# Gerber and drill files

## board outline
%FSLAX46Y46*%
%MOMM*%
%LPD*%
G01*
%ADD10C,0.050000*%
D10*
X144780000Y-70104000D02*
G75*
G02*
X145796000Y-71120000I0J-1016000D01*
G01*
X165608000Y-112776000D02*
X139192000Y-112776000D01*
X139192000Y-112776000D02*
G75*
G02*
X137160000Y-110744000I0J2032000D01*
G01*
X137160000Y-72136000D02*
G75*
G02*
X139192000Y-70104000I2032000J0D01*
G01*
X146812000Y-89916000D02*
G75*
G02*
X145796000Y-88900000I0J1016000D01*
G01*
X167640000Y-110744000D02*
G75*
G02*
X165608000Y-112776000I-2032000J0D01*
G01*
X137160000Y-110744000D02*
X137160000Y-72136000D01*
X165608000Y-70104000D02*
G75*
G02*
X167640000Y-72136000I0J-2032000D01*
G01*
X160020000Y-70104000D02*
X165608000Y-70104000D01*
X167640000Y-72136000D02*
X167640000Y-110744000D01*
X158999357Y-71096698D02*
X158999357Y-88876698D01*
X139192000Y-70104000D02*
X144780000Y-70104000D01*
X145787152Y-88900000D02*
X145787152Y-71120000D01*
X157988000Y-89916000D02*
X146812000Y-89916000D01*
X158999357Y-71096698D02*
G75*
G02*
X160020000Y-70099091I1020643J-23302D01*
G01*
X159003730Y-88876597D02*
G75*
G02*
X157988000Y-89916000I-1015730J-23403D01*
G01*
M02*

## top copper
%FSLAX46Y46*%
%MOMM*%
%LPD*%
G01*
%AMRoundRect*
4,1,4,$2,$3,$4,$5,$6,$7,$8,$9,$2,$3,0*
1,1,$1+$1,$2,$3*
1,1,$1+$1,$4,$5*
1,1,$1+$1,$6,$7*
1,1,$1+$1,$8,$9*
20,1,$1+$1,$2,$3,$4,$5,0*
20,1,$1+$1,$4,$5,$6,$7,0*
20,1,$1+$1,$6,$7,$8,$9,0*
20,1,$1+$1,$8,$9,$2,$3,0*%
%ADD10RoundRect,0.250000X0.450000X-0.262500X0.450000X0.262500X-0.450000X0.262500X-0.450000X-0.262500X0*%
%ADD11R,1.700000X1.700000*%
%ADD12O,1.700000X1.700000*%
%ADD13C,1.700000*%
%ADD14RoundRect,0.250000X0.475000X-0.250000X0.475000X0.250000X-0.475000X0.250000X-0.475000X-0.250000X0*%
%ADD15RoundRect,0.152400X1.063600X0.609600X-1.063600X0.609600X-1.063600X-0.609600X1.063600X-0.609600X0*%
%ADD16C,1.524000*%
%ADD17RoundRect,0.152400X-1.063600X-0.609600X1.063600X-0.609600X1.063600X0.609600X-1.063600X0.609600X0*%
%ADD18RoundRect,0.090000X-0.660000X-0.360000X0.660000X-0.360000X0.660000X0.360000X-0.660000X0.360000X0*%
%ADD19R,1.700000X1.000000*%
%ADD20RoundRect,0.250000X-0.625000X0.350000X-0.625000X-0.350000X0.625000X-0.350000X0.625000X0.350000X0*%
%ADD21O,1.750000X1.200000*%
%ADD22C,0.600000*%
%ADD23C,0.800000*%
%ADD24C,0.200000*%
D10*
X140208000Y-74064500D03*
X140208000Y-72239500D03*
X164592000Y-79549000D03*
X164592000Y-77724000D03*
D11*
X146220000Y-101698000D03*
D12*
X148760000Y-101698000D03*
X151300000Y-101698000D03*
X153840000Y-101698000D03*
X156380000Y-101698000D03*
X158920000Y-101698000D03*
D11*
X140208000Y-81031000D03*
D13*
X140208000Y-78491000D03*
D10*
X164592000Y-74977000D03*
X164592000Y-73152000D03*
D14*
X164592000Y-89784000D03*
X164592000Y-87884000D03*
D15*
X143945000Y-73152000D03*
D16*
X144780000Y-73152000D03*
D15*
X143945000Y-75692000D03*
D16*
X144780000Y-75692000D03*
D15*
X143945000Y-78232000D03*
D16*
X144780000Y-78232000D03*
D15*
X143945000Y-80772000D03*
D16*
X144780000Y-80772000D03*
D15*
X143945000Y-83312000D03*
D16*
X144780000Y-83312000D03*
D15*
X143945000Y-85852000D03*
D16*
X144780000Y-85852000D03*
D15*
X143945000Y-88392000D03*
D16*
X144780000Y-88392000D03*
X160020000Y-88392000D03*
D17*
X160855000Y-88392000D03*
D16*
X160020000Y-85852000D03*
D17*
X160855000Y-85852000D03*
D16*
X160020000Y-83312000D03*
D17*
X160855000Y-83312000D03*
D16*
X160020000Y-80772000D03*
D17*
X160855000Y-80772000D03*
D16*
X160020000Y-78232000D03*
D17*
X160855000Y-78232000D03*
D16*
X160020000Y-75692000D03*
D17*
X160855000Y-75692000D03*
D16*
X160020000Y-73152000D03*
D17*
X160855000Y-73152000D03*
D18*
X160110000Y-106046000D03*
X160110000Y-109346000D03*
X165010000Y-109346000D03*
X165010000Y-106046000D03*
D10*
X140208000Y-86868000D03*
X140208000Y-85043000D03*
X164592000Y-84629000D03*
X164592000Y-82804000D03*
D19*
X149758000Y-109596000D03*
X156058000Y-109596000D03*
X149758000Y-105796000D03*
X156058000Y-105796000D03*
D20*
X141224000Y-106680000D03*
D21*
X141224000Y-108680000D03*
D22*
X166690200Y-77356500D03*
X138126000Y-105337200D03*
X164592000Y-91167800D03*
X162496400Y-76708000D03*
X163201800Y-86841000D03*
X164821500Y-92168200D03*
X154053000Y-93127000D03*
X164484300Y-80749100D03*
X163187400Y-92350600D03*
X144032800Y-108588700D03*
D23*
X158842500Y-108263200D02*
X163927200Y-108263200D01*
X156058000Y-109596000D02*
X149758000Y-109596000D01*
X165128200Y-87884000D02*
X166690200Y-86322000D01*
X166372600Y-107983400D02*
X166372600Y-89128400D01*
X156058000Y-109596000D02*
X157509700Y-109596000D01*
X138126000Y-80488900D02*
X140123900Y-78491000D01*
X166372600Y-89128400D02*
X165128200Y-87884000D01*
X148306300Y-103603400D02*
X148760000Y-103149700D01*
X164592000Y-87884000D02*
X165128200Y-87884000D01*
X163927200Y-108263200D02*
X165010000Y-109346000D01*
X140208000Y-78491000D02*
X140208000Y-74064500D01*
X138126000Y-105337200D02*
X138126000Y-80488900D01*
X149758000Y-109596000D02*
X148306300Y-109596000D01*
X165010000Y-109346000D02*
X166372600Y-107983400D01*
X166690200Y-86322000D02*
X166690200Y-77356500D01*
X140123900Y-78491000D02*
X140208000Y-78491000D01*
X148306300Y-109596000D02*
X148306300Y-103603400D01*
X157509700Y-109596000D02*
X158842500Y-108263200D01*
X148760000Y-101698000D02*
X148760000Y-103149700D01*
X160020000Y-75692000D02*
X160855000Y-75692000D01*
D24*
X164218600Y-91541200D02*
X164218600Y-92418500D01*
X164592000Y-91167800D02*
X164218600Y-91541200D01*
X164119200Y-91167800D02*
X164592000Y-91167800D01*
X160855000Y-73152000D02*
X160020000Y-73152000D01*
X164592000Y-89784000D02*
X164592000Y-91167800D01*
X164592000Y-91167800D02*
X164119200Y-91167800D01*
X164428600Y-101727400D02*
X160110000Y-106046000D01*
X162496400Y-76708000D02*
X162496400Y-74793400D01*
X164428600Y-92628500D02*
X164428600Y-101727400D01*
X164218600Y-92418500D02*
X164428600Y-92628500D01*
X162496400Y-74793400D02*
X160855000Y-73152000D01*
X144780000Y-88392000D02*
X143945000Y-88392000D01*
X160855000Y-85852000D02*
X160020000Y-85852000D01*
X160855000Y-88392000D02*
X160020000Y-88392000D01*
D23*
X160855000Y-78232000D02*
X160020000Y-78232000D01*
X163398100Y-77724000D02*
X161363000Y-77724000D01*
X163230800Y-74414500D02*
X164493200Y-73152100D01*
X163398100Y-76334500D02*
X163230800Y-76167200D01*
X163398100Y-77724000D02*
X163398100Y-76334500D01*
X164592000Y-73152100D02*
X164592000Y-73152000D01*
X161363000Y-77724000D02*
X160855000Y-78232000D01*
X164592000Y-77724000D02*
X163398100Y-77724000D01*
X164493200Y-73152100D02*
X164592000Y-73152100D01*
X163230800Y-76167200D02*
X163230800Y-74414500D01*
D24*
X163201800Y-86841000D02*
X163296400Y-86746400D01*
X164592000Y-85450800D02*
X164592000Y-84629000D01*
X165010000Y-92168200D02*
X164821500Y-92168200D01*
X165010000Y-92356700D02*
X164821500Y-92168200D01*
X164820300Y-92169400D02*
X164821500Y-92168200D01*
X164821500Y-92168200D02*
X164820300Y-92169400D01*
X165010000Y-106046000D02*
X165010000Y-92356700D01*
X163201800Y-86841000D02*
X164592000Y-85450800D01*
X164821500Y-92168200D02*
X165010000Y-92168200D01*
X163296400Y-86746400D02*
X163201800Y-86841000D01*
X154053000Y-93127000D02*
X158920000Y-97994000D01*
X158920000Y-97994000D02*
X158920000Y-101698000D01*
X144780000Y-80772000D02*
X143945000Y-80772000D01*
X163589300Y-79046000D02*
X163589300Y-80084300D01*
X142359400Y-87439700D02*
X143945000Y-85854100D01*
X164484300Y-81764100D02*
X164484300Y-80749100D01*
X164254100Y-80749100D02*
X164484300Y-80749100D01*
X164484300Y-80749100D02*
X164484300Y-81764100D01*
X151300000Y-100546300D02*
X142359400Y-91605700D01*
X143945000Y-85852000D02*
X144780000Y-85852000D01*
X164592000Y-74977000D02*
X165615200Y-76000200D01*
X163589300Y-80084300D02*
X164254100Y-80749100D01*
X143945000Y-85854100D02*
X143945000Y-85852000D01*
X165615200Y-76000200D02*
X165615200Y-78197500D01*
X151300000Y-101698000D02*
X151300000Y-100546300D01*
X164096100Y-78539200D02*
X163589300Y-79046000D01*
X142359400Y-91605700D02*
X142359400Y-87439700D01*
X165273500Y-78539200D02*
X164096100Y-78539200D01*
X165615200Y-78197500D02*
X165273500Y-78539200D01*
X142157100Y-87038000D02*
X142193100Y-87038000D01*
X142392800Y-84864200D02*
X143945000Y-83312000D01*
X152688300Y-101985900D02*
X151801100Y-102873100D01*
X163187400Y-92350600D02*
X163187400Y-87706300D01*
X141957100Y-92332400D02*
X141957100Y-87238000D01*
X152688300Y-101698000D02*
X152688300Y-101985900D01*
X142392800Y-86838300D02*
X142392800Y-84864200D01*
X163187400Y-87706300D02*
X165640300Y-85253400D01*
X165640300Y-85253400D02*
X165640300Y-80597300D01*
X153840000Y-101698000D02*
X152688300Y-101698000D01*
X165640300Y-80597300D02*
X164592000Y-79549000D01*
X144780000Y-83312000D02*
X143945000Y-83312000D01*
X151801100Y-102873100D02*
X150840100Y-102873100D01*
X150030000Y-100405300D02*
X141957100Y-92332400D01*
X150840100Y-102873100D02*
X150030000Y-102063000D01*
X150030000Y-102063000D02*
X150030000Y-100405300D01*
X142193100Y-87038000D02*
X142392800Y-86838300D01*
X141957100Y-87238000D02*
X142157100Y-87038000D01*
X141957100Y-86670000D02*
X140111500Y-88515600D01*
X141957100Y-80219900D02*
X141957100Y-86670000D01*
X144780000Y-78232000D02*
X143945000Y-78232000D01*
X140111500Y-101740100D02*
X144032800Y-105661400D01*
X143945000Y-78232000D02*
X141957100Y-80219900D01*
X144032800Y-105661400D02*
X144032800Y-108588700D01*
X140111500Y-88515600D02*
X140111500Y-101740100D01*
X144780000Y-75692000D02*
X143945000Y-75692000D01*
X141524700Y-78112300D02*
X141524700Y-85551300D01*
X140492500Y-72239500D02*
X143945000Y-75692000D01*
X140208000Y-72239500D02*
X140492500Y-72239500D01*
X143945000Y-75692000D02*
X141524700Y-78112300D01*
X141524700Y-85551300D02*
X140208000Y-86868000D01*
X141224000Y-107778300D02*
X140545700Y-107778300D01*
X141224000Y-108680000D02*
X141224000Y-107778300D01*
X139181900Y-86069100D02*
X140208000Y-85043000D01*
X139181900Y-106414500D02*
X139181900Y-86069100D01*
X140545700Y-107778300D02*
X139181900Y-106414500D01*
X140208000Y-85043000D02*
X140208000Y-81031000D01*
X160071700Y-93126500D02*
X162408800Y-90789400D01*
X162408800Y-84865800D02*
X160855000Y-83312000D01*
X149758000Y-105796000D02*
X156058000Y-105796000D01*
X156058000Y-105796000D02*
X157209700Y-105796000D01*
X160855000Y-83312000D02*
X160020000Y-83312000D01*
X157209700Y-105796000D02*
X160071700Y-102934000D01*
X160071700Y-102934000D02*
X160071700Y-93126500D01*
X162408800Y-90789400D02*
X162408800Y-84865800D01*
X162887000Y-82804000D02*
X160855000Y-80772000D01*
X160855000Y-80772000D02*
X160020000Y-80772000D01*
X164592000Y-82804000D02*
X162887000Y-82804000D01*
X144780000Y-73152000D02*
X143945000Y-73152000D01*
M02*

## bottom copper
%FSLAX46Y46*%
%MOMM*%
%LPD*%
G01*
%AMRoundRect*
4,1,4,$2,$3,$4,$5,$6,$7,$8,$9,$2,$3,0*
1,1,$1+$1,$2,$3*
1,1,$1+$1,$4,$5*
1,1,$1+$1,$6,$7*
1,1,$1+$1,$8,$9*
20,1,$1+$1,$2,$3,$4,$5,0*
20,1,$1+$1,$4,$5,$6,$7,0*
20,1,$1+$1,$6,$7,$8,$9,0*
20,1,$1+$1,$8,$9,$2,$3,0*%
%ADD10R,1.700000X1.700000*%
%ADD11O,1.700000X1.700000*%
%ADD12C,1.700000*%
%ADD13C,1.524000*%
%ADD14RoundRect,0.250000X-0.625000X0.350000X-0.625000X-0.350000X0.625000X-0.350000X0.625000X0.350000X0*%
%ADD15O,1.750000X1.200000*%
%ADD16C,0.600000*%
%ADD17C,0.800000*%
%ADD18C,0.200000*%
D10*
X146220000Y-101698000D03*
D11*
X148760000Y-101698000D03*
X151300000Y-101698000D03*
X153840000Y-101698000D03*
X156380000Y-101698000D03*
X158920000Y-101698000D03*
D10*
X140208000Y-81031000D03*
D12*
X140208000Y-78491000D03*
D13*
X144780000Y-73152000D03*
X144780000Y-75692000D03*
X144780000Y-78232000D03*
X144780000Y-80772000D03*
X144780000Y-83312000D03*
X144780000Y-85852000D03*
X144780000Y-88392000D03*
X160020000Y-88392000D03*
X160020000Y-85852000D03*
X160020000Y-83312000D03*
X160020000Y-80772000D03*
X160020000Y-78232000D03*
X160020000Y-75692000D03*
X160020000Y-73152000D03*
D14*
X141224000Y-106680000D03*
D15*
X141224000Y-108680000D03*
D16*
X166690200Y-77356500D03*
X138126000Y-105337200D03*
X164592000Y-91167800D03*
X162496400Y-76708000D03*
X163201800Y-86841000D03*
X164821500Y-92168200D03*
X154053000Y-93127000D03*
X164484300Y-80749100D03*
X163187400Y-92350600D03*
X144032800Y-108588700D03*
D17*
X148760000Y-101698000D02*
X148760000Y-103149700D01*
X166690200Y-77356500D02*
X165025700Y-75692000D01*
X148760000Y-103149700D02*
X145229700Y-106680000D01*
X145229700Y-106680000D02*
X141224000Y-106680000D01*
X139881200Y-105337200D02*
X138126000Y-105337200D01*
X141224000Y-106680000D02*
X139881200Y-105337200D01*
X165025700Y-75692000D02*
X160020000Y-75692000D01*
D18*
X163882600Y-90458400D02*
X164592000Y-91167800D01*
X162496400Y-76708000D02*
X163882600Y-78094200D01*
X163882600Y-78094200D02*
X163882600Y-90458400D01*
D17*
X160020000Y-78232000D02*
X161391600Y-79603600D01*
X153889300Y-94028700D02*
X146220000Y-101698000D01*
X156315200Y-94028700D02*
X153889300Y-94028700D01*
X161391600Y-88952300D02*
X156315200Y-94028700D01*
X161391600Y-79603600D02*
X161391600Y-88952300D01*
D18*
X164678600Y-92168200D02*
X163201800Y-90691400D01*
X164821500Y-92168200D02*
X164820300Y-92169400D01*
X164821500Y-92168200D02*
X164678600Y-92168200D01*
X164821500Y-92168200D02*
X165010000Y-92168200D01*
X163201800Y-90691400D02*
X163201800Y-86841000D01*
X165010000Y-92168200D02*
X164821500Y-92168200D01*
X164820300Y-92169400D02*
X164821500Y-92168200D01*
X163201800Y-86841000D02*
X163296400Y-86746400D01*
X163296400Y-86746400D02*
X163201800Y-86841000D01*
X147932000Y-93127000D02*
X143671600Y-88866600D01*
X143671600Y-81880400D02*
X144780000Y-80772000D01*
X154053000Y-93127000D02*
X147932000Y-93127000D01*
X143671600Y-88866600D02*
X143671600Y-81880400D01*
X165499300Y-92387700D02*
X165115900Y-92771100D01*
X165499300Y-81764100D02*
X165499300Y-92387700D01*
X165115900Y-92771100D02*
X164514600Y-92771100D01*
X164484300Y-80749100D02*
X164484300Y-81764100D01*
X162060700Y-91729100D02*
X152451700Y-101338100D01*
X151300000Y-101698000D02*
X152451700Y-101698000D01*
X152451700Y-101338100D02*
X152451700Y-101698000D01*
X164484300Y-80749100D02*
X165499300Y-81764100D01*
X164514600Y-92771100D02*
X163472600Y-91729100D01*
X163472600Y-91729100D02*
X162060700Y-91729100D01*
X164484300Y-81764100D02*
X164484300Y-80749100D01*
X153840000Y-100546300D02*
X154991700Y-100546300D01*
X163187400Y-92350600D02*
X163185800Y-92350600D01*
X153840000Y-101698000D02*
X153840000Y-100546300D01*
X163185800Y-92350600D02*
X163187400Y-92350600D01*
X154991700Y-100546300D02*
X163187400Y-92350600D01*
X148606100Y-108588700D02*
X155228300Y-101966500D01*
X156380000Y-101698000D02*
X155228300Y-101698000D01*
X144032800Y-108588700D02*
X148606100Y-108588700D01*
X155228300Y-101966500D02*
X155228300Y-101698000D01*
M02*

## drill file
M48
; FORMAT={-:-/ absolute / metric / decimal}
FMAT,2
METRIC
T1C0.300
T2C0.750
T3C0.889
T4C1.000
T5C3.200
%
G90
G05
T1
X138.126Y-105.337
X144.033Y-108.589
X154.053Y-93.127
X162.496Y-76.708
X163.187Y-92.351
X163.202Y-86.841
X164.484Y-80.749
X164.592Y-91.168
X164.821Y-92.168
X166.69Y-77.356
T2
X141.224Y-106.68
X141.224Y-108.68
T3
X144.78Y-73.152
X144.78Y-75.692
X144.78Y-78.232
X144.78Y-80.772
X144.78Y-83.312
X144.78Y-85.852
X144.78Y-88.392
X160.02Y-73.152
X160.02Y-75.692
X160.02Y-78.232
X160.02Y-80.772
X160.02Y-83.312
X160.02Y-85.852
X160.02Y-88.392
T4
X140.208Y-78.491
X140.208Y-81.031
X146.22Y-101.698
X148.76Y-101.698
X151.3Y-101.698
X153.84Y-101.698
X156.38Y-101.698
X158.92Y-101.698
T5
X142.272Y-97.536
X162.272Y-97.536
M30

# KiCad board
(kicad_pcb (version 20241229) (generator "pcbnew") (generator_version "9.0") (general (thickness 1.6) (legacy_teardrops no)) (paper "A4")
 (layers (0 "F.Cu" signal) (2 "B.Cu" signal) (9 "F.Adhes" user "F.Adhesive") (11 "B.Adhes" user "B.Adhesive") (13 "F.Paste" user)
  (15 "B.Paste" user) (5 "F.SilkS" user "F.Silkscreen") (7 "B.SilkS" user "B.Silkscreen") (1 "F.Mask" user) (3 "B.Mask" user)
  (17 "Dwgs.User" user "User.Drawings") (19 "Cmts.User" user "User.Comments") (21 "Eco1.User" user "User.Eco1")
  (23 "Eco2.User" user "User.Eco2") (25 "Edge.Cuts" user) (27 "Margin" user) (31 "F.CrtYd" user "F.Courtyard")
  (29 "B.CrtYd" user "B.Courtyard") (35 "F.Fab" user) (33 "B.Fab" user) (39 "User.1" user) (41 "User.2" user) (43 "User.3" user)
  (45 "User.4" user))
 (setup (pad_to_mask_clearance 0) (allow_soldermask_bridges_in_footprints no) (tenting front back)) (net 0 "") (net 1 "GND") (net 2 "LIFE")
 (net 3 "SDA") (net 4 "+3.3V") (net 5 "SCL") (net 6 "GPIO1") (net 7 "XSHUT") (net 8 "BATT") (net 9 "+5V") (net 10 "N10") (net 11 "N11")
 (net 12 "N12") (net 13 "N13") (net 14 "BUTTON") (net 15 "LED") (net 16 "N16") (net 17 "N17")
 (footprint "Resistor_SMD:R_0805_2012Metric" (layer "F.Cu") (at 140.208 73.152 90)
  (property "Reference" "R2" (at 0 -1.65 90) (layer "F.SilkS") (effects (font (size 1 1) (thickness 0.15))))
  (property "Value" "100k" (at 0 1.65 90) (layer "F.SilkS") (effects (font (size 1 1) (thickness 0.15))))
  (pad "1" smd roundrect (at -0.9125 0 90) (size 1.025 1.4) (layers "F.Cu" "F.Mask" "F.Paste") (roundrect_rratio 0.243902) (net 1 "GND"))
  (pad "2" smd roundrect (at 0.9125 0 90) (size 1.025 1.4) (layers "F.Cu" "F.Mask" "F.Paste") (roundrect_rratio 0.243902) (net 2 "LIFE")))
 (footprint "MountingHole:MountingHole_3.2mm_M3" (layer "F.Cu") (at 162.272 97.536)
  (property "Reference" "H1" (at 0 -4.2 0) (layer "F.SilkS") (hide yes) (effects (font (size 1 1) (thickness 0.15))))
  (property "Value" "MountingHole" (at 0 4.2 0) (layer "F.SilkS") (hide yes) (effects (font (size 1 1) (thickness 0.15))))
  (pad "" np_thru_hole circle (at 0 0) (size 3.2 3.2) (drill 3.2) (layers "*.Cu" "*.Mask")))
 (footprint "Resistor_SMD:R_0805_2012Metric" (layer "F.Cu") (at 164.592 78.6365 90)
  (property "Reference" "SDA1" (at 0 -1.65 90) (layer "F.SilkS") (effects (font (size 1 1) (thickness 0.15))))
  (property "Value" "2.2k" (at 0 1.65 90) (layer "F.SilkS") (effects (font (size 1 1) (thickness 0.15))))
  (pad "1" smd roundrect (at -0.9125 0 90) (size 1.025 1.4) (layers "F.Cu" "F.Mask" "F.Paste") (roundrect_rratio 0.243902) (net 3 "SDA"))
  (pad "2" smd roundrect (at 0.9125 0 90) (size 1.025 1.4) (layers "F.Cu" "F.Mask" "F.Paste") (roundrect_rratio 0.243902) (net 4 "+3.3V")))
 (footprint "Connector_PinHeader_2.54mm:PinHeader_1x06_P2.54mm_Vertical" (layer "F.Cu") (at 146.22 101.698 90)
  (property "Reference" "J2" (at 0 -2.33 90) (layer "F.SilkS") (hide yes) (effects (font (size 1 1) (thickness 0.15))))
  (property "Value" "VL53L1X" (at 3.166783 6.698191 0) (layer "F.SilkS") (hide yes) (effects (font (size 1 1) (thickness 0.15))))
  (pad "1" thru_hole rect (at 0 0 90) (size 1.7 1.7) (drill 1) (layers "*.Cu" "*.Mask") (remove_unused_layers no) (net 4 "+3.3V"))
  (pad "2" thru_hole oval (at 0 2.54 90) (size 1.7 1.7) (drill 1) (layers "*.Cu" "*.Mask") (remove_unused_layers no) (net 1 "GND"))
  (pad "3" thru_hole oval (at 0 5.08 90) (size 1.7 1.7) (drill 1) (layers "*.Cu" "*.Mask") (remove_unused_layers no) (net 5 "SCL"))
  (pad "4" thru_hole oval (at 0 7.62 90) (size 1.7 1.7) (drill 1) (layers "*.Cu" "*.Mask") (remove_unused_layers no) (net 3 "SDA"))
  (pad "5" thru_hole oval (at 0 10.16 90) (size 1.7 1.7) (drill 1) (layers "*.Cu" "*.Mask") (remove_unused_layers no) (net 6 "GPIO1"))
  (pad "6" thru_hole oval (at 0 12.7 90) (size 1.7 1.7) (drill 1) (layers "*.Cu" "*.Mask") (remove_unused_layers no) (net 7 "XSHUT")))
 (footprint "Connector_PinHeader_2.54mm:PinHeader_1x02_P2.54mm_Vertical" (layer "F.Cu") (at 140.208 81.031 180)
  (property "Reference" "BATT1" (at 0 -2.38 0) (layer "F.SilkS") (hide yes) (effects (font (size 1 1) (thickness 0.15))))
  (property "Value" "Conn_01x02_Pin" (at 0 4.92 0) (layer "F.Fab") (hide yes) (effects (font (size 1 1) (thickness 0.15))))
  (pad "1" thru_hole rect (at 0 0 180) (size 1.7 1.7) (drill 1) (layers "*.Cu" "*.Mask") (remove_unused_layers no) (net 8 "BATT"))
  (pad "2" thru_hole circle (at 0 2.54 180) (size 1.7 1.7) (drill 1) (layers "*.Cu" "*.Mask") (remove_unused_layers no) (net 1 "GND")))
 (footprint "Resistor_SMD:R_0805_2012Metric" (layer "F.Cu") (at 164.592 74.0645 90)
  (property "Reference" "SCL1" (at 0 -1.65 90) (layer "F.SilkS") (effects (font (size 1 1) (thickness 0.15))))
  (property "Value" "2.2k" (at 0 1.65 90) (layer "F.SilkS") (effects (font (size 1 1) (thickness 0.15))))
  (pad "1" smd roundrect (at -0.9125 0 90) (size 1.025 1.4) (layers "F.Cu" "F.Mask" "F.Paste") (roundrect_rratio 0.243902) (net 5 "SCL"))
  (pad "2" smd roundrect (at 0.9125 0 90) (size 1.025 1.4) (layers "F.Cu" "F.Mask" "F.Paste") (roundrect_rratio 0.243902) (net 4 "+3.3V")))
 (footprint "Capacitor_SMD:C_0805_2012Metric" (layer "F.Cu") (at 164.592 88.834 90)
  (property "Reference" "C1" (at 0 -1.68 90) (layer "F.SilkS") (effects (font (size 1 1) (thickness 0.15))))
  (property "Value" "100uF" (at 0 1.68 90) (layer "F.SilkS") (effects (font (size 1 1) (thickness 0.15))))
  (pad "1" smd roundrect (at -0.95 0 90) (size 1 1.45) (layers "F.Cu" "F.Mask" "F.Paste") (roundrect_rratio 0.25) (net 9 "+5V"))
  (pad "2" smd roundrect (at 0.95 0 90) (size 1 1.45) (layers "F.Cu" "F.Mask" "F.Paste") (roundrect_rratio 0.25) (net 1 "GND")))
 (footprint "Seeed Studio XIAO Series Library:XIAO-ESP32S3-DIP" (layer "F.Cu") (at 152.4 80.772)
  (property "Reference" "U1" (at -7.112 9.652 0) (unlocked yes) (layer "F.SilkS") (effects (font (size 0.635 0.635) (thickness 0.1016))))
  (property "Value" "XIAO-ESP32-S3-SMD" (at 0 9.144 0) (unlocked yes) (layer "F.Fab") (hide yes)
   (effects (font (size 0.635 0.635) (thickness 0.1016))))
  (pad "1" smd roundrect (at -8.455 -7.62 180) (size 2.432 1.524) (layers "F.Cu" "F.Mask") (roundrect_rratio 0.1) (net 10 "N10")
   (thermal_bridge_angle 45))
  (pad "1" thru_hole circle (at -7.62 -7.62 180) (size 1.524 1.524) (drill 0.889) (layers "*.Cu" "*.Mask") (remove_unused_layers no)
   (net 10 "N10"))
  (pad "2" smd roundrect (at -8.455 -5.08 180) (size 2.432 1.524) (layers "F.Cu" "F.Mask") (roundrect_rratio 0.1) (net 2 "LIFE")
   (thermal_bridge_angle 45))
  (pad "2" thru_hole circle (at -7.62 -5.08 180) (size 1.524 1.524) (drill 0.889) (layers "*.Cu" "*.Mask") (remove_unused_layers no)
   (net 2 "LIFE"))
  (pad "3" smd roundrect (at -8.455 -2.54 180) (size 2.432 1.524) (layers "F.Cu" "F.Mask") (roundrect_rratio 0.1) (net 6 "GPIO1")
   (thermal_bridge_angle 45))
  (pad "3" thru_hole circle (at -7.62 -2.54 180) (size 1.524 1.524) (drill 0.889) (layers "*.Cu" "*.Mask") (remove_unused_layers no)
   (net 6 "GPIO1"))
  (pad "4" smd roundrect (at -8.455 0 180) (size 2.432 1.524) (layers "F.Cu" "F.Mask") (roundrect_rratio 0.1) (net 7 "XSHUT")
   (thermal_bridge_angle 45))
  (pad "4" thru_hole circle (at -7.62 0 180) (size 1.524 1.524) (drill 0.889) (layers "*.Cu" "*.Mask") (remove_unused_layers no)
   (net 7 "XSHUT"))
  (pad "5" smd roundrect (at -8.455 2.54 180) (size 2.432 1.524) (layers "F.Cu" "F.Mask") (roundrect_rratio 0.1) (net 3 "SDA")
   (thermal_bridge_angle 45))
  (pad "5" thru_hole circle (at -7.62 2.54 180) (size 1.524 1.524) (drill 0.889) (layers "*.Cu" "*.Mask") (remove_unused_layers no)
   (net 3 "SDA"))
  (pad "6" smd roundrect (at -8.455 5.08 180) (size 2.432 1.524) (layers "F.Cu" "F.Mask") (roundrect_rratio 0.1) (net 5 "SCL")
   (thermal_bridge_angle 45))
  (pad "6" thru_hole circle (at -7.62 5.08 180) (size 1.524 1.524) (drill 0.889) (layers "*.Cu" "*.Mask") (remove_unused_layers no)
   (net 5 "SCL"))
  (pad "7" smd roundrect (at -8.455 7.62 180) (size 2.432 1.524) (layers "F.Cu" "F.Mask") (roundrect_rratio 0.1) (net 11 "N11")
   (thermal_bridge_angle 45))
  (pad "7" thru_hole circle (at -7.62 7.62 180) (size 1.524 1.524) (drill 0.889) (layers "*.Cu" "*.Mask") (remove_unused_layers no)
   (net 11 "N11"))
  (pad "8" thru_hole circle (at 7.62 7.62) (size 1.524 1.524) (drill 0.889) (layers "*.Cu" "*.Mask") (remove_unused_layers no)
   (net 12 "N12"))
  (pad "8" smd roundrect (at 8.455 7.62) (size 2.432 1.524) (layers "F.Cu" "F.Mask") (roundrect_rratio 0.1) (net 12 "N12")
   (thermal_bridge_angle 45))
  (pad "9" thru_hole circle (at 7.62 5.08) (size 1.524 1.524) (drill 0.889) (layers "*.Cu" "*.Mask") (remove_unused_layers no)
   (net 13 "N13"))
  (pad "9" smd roundrect (at 8.455 5.08) (size 2.432 1.524) (layers "F.Cu" "F.Mask") (roundrect_rratio 0.1) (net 13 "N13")
   (thermal_bridge_angle 45))
  (pad "10" thru_hole circle (at 7.62 2.54) (size 1.524 1.524) (drill 0.889) (layers "*.Cu" "*.Mask") (remove_unused_layers no)
   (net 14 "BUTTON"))
  (pad "10" smd roundrect (at 8.455 2.54) (size 2.432 1.524) (layers "F.Cu" "F.Mask") (roundrect_rratio 0.1) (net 14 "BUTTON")
   (thermal_bridge_angle 45))
  (pad "11" thru_hole circle (at 7.62 0) (size 1.524 1.524) (drill 0.889) (layers "*.Cu" "*.Mask") (remove_unused_layers no) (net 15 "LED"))
  (pad "11" smd roundrect (at 8.455 0) (size 2.432 1.524) (layers "F.Cu" "F.Mask") (roundrect_rratio 0.1) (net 15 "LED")
   (thermal_bridge_angle 45))
  (pad "12" thru_hole circle (at 7.62 -2.54) (size 1.524 1.524) (drill 0.889) (layers "*.Cu" "*.Mask") (remove_unused_layers no)
   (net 4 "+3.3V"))
  (pad "12" smd roundrect (at 8.455 -2.54) (size 2.432 1.524) (layers "F.Cu" "F.Mask") (roundrect_rratio 0.1) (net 4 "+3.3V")
   (thermal_bridge_angle 45))
  (pad "13" thru_hole circle (at 7.62 -5.08) (size 1.524 1.524) (drill 0.889) (layers "*.Cu" "*.Mask") (remove_unused_layers no)
   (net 1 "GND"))
  (pad "13" smd roundrect (at 8.455 -5.08) (size 2.432 1.524) (layers "F.Cu" "F.Mask") (roundrect_rratio 0.1) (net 1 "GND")
   (thermal_bridge_angle 45))
  (pad "14" thru_hole circle (at 7.62 -7.62) (size 1.524 1.524) (drill 0.889) (layers "*.Cu" "*.Mask") (remove_unused_layers no)
   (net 9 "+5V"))
  (pad "14" smd roundrect (at 8.455 -7.62) (size 2.432 1.524) (layers "F.Cu" "F.Mask") (roundrect_rratio 0.1) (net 9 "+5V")
   (thermal_bridge_angle 45)))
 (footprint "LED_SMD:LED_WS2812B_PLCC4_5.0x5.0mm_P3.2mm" (layer "F.Cu") (at 162.56 107.696)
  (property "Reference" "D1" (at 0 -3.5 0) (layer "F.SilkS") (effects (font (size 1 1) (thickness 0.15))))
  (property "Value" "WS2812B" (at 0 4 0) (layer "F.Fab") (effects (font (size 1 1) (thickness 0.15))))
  (pad "1" smd roundrect (at -2.45 -1.65) (size 1.5 0.9) (layers "F.Cu" "F.Mask" "F.Paste") (roundrect_rratio 0.1) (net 9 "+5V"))
  (pad "2" smd roundrect (at -2.45 1.65) (size 1.5 0.9) (layers "F.Cu" "F.Mask" "F.Paste") (roundrect_rratio 0.1) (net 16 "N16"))
  (pad "3" smd roundrect (at 2.45 1.65) (size 1.5 0.9) (layers "F.Cu" "F.Mask" "F.Paste") (roundrect_rratio 0.1) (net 1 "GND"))
  (pad "4" smd roundrect (at 2.45 -1.65) (size 1.5 0.9) (layers "F.Cu" "F.Mask" "F.Paste") (roundrect_rratio 0.1) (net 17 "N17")))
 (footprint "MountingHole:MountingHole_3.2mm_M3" (layer "F.Cu") (at 142.272 97.536)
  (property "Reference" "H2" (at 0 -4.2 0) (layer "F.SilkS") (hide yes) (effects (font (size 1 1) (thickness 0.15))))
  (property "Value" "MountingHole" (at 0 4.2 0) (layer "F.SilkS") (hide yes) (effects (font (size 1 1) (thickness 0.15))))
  (pad "" np_thru_hole circle (at 0 0) (size 3.2 3.2) (drill 3.2) (layers "*.Cu" "*.Mask")))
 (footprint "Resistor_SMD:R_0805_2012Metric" (layer "F.Cu") (at 140.208 85.9555 90)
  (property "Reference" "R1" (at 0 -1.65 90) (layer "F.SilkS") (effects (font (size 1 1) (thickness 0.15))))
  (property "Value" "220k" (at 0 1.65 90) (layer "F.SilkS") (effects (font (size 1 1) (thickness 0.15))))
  (pad "1" smd roundrect (at -0.9125 0 90) (size 1.025 1.4) (layers "F.Cu" "F.Mask" "F.Paste") (roundrect_rratio 0.243902) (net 2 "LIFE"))
  (pad "2" smd roundrect (at 0.9125 0 90) (size 1.025 1.4) (layers "F.Cu" "F.Mask" "F.Paste") (roundrect_rratio 0.243902) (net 8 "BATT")))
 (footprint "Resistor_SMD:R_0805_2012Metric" (layer "F.Cu") (at 164.592 83.7165 90)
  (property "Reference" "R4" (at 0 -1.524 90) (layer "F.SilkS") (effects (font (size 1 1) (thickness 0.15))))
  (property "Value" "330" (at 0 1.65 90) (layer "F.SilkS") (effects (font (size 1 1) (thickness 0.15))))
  (pad "1" smd roundrect (at -0.9125 0 90) (size 1.025 1.4) (layers "F.Cu" "F.Mask" "F.Paste") (roundrect_rratio 0.243902) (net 17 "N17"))
  (pad "2" smd roundrect (at 0.9125 0 90) (size 1.025 1.4) (layers "F.Cu" "F.Mask" "F.Paste") (roundrect_rratio 0.243902) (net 15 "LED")))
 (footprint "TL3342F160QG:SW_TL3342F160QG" (layer "F.Cu") (at 152.908 107.696)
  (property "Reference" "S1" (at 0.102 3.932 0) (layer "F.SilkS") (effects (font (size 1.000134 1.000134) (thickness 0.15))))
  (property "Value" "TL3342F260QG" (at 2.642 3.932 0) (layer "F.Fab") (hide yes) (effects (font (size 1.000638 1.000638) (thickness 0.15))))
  (pad "1" smd rect (at -3.15 1.9) (size 1.7 1) (layers "F.Cu" "F.Mask" "F.Paste") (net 1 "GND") (solder_mask_margin 0.102))
  (pad "2" smd rect (at 3.15 1.9) (size 1.7 1) (layers "F.Cu" "F.Mask" "F.Paste") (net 1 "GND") (solder_mask_margin 0.102))
  (pad "3" smd rect (at -3.15 -1.9) (size 1.7 1) (layers "F.Cu" "F.Mask" "F.Paste") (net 14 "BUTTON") (solder_mask_margin 0.102))
  (pad "4" smd rect (at 3.15 -1.9) (size 1.7 1) (layers "F.Cu" "F.Mask" "F.Paste") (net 14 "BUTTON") (solder_mask_margin 0.102)))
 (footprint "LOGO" (layer "B.Cu") (at 152.4 95.504 180)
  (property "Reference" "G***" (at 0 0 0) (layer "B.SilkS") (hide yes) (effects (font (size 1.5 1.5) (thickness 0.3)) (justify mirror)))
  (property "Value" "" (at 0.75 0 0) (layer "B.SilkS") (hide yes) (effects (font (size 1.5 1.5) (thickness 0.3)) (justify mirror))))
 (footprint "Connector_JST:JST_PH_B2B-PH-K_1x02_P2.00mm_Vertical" (layer "B.Cu") (at 141.224 106.68 -90)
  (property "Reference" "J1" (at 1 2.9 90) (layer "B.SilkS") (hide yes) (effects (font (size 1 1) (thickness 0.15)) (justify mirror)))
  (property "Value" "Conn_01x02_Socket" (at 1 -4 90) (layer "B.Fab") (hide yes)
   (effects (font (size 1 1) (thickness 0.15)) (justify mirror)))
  (pad "1" thru_hole roundrect (at 0 0 270) (size 1.2 1.75) (drill 0.75) (layers "*.Cu" "*.Mask") (remove_unused_layers no)
   (roundrect_rratio 0.208333) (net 1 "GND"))
  (pad "2" thru_hole oval (at 2 0 270) (size 1.2 1.75) (drill 0.75) (layers "*.Cu" "*.Mask") (remove_unused_layers no) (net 8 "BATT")))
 (gr_arc (start 144.78 70.104) (mid 145.49842 70.40158) (end 145.796 71.12) (stroke (width 0.05) (type default)) (layer "Edge.Cuts"))
 (gr_line (start 165.608 112.776) (end 139.192 112.776) (stroke (width 0.05) (type default)) (layer "Edge.Cuts"))
 (gr_arc (start 139.192 112.776) (mid 137.755159 112.180841) (end 137.16 110.744) (stroke (width 0.05) (type default)) (layer "Edge.Cuts"))
 (gr_arc (start 137.16 72.136) (mid 137.755159 70.699159) (end 139.192 70.104) (stroke (width 0.05) (type default)) (layer "Edge.Cuts"))
 (gr_arc (start 146.812 89.916) (mid 146.09358 89.61842) (end 145.796 88.9) (stroke (width 0.05) (type default)) (layer "Edge.Cuts"))
 (gr_arc (start 167.64 110.744) (mid 167.044841 112.180841) (end 165.608 112.776) (stroke (width 0.05) (type default)) (layer "Edge.Cuts"))
 (gr_line (start 137.16 110.744) (end 137.16 72.136) (stroke (width 0.05) (type default)) (layer "Edge.Cuts"))
 (gr_arc (start 165.608 70.104) (mid 167.044841 70.699159) (end 167.64 72.136) (stroke (width 0.05) (type default)) (layer "Edge.Cuts"))
 (gr_line (start 160.02 70.104) (end 165.608 70.104) (stroke (width 0.05) (type default)) (layer "Edge.Cuts"))
 (gr_line (start 167.64 72.136) (end 167.64 110.744) (stroke (width 0.05) (type default)) (layer "Edge.Cuts"))
 (gr_line (start 158.999357 71.096698) (end 158.999357 88.876698) (stroke (width 0.05) (type default)) (layer "Edge.Cuts"))
 (gr_line (start 139.192 70.104) (end 144.78 70.104) (stroke (width 0.05) (type default)) (layer "Edge.Cuts"))
 (gr_line (start 145.787152 88.9) (end 145.787152 71.12) (stroke (width 0.05) (type default)) (layer "Edge.Cuts"))
 (gr_line (start 157.988 89.916) (end 146.812 89.916) (stroke (width 0.05) (type default)) (layer "Edge.Cuts"))
 (gr_arc (start 158.999357 71.096698) (mid 159.306394 70.389916) (end 160.02 70.099091) (stroke (width 0.05) (type default))
  (layer "Edge.Cuts"))
 (gr_arc (start 159.00373 88.876597) (mid 158.714647 89.610098) (end 157.988 89.916) (stroke (width 0.05) (type default))
  (layer "Edge.Cuts"))
 (segment (start 158.8425 108.2632) (end 163.9272 108.2632) (width 0.8) (layer "F.Cu") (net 1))
 (segment (start 156.058 109.596) (end 149.758 109.596) (width 0.8) (layer "F.Cu") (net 1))
 (segment (start 165.1282 87.884) (end 166.6902 86.322) (width 0.8) (layer "F.Cu") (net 1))
 (segment (start 166.3726 107.9834) (end 166.3726 89.1284) (width 0.8) (layer "F.Cu") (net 1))
 (segment (start 156.058 109.596) (end 157.5097 109.596) (width 0.8) (layer "F.Cu") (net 1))
 (segment (start 138.126 80.4889) (end 140.1239 78.491) (width 0.8) (layer "F.Cu") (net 1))
 (segment (start 166.3726 89.1284) (end 165.1282 87.884) (width 0.8) (layer "F.Cu") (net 1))
 (segment (start 148.3063 103.6034) (end 148.76 103.1497) (width 0.8) (layer "F.Cu") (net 1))
 (segment (start 164.592 87.884) (end 165.1282 87.884) (width 0.8) (layer "F.Cu") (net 1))
 (segment (start 163.9272 108.2632) (end 165.01 109.346) (width 0.8) (layer "F.Cu") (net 1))
 (segment (start 140.208 78.491) (end 140.208 74.0645) (width 0.8) (layer "F.Cu") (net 1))
 (segment (start 138.126 105.3372) (end 138.126 80.4889) (width 0.8) (layer "F.Cu") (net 1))
 (segment (start 149.758 109.596) (end 148.3063 109.596) (width 0.8) (layer "F.Cu") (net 1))
 (segment (start 165.01 109.346) (end 166.3726 107.9834) (width 0.8) (layer "F.Cu") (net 1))
 (segment (start 166.6902 86.322) (end 166.6902 77.3565) (width 0.8) (layer "F.Cu") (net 1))
 (segment (start 140.1239 78.491) (end 140.208 78.491) (width 0.8) (layer "F.Cu") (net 1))
 (segment (start 148.3063 109.596) (end 148.3063 103.6034) (width 0.8) (layer "F.Cu") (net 1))
 (segment (start 157.5097 109.596) (end 158.8425 108.2632) (width 0.8) (layer "F.Cu") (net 1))
 (segment (start 148.76 101.698) (end 148.76 103.1497) (width 0.8) (layer "F.Cu") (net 1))
 (segment (start 160.02 75.692) (end 160.855 75.692) (width 0.8) (layer "F.Cu") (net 1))
 (via (at 166.6902 77.3565) (size 0.6) (drill 0.3) (layers "F.Cu" "B.Cu") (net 1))
 (via (at 138.126 105.3372) (size 0.6) (drill 0.3) (layers "F.Cu" "B.Cu") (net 1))
 (segment (start 148.76 101.698) (end 148.76 103.1497) (width 0.8) (layer "B.Cu") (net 1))
 (segment (start 166.6902 77.3565) (end 165.0257 75.692) (width 0.8) (layer "B.Cu") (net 1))
 (segment (start 148.76 103.1497) (end 145.2297 106.68) (width 0.8) (layer "B.Cu") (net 1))
 (segment (start 145.2297 106.68) (end 141.224 106.68) (width 0.8) (layer "B.Cu") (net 1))
 (segment (start 139.8812 105.3372) (end 138.126 105.3372) (width 0.8) (layer "B.Cu") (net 1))
 (segment (start 141.224 106.68) (end 139.8812 105.3372) (width 0.8) (layer "B.Cu") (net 1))
 (segment (start 165.0257 75.692) (end 160.02 75.692) (width 0.8) (layer "B.Cu") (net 1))
 (segment (start 164.2186 91.5412) (end 164.2186 92.4185) (width 0.2) (layer "F.Cu") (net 9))
 (segment (start 164.592 91.1678) (end 164.2186 91.5412) (width 0.2) (layer "F.Cu") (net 9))
 (segment (start 164.1192 91.1678) (end 164.592 91.1678) (width 0.2) (layer "F.Cu") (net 9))
 (segment (start 160.855 73.152) (end 160.02 73.152) (width 0.2) (layer "F.Cu") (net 9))
 (segment (start 164.592 89.784) (end 164.592 91.1678) (width 0.2) (layer "F.Cu") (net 9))
 (segment (start 164.592 91.1678) (end 164.1192 91.1678) (width 0.2) (layer "F.Cu") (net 9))
 (segment (start 164.4286 101.7274) (end 160.11 106.046) (width 0.2) (layer "F.Cu") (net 9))
 (segment (start 162.4964 76.708) (end 162.4964 74.7934) (width 0.2) (layer "F.Cu") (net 9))
 (segment (start 164.4286 92.6285) (end 164.4286 101.7274) (width 0.2) (layer "F.Cu") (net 9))
 (segment (start 164.2186 92.4185) (end 164.4286 92.6285) (width 0.2) (layer "F.Cu") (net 9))
 (segment (start 162.4964 74.7934) (end 160.855 73.152) (width 0.2) (layer "F.Cu") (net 9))
 (via (at 164.592 91.1678) (size 0.6) (drill 0.3) (layers "F.Cu" "B.Cu") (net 9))
 (via (at 162.4964 76.708) (size 0.6) (drill 0.3) (layers "F.Cu" "B.Cu") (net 9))
 (segment (start 163.8826 90.4584) (end 164.592 91.1678) (width 0.2) (layer "B.Cu") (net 9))
 (segment (start 162.4964 76.708) (end 163.8826 78.0942) (width 0.2) (layer "B.Cu") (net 9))
 (segment (start 163.8826 78.0942) (end 163.8826 90.4584) (width 0.2) (layer "B.Cu") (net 9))
 (segment (start 144.78 88.392) (end 143.945 88.392) (width 0.2) (layer "F.Cu") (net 11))
 (segment (start 160.855 85.852) (end 160.02 85.852) (width 0.2) (layer "F.Cu") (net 13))
 (segment (start 160.855 88.392) (end 160.02 88.392) (width 0.2) (layer "F.Cu") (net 12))
 (segment (start 160.855 78.232) (end 160.02 78.232) (width 0.8) (layer "F.Cu") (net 4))
 (segment (start 163.3981 77.724) (end 161.363 77.724) (width 0.8) (layer "F.Cu") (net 4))
 (segment (start 163.2308 74.4145) (end 164.4932 73.1521) (width 0.8) (layer "F.Cu") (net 4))
 (segment (start 163.3981 76.3345) (end 163.2308 76.1672) (width 0.8) (layer "F.Cu") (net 4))
 (segment (start 163.3981 77.724) (end 163.3981 76.3345) (width 0.8) (layer "F.Cu") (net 4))
 (segment (start 164.592 73.1521) (end 164.592 73.152) (width 0.8) (layer "F.Cu") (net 4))
 (segment (start 161.363 77.724) (end 160.855 78.232) (width 0.8) (layer "F.Cu") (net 4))
 (segment (start 164.592 77.724) (end 163.3981 77.724) (width 0.8) (layer "F.Cu") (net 4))
 (segment (start 164.4932 73.1521) (end 164.592 73.1521) (width 0.8) (layer "F.Cu") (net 4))
 (segment (start 163.2308 76.1672) (end 163.2308 74.4145) (width 0.8) (layer "F.Cu") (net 4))
 (segment (start 160.02 78.232) (end 161.3916 79.6036) (width 0.8) (layer "B.Cu") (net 4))
 (segment (start 153.8893 94.0287) (end 146.22 101.698) (width 0.8) (layer "B.Cu") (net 4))
 (segment (start 156.3152 94.0287) (end 153.8893 94.0287) (width 0.8) (layer "B.Cu") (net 4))
 (segment (start 161.3916 88.9523) (end 156.3152 94.0287) (width 0.8) (layer "B.Cu") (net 4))
 (segment (start 161.3916 79.6036) (end 161.3916 88.9523) (width 0.8) (layer "B.Cu") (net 4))
 (segment (start 163.2018 86.841) (end 163.2964 86.7464) (width 0.2) (layer "F.Cu") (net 17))
 (segment (start 164.592 85.4508) (end 164.592 84.629) (width 0.2) (layer "F.Cu") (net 17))
 (segment (start 165.01 92.1682) (end 164.8215 92.1682) (width 0.2) (layer "F.Cu") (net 17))
 (segment (start 165.01 92.3567) (end 164.8215 92.1682) (width 0.2) (layer "F.Cu") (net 17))
 (segment (start 164.8203 92.1694) (end 164.8215 92.1682) (width 0.2) (layer "F.Cu") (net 17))
 (segment (start 164.8215 92.1682) (end 164.8203 92.1694) (width 0.2) (layer "F.Cu") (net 17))
 (segment (start 165.01 106.046) (end 165.01 92.3567) (width 0.2) (layer "F.Cu") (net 17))
 (segment (start 163.2018 86.841) (end 164.592 85.4508) (width 0.2) (layer "F.Cu") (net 17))
 (segment (start 164.8215 92.1682) (end 165.01 92.1682) (width 0.2) (layer "F.Cu") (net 17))
 (segment (start 163.2964 86.7464) (end 163.2018 86.841) (width 0.2) (layer "F.Cu") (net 17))
 (via (at 163.2018 86.841) (size 0.6) (drill 0.3) (layers "F.Cu" "B.Cu") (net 17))
 (via (at 164.8215 92.1682) (size 0.6) (drill 0.3) (layers "F.Cu" "B.Cu") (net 17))
 (segment (start 164.6786 92.1682) (end 163.2018 90.6914) (width 0.2) (layer "B.Cu") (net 17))
 (segment (start 164.8215 92.1682) (end 164.8203 92.1694) (width 0.2) (layer "B.Cu") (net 17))
 (segment (start 164.8215 92.1682) (end 164.6786 92.1682) (width 0.2) (layer "B.Cu") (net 17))
 (segment (start 164.8215 92.1682) (end 165.01 92.1682) (width 0.2) (layer "B.Cu") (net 17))
 (segment (start 163.2018 90.6914) (end 163.2018 86.841) (width 0.2) (layer "B.Cu") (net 17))
 (segment (start 165.01 92.1682) (end 164.8215 92.1682) (width 0.2) (layer "B.Cu") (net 17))
 (segment (start 164.8203 92.1694) (end 164.8215 92.1682) (width 0.2) (layer "B.Cu") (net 17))
 (segment (start 163.2018 86.841) (end 163.2964 86.7464) (width 0.2) (layer "B.Cu") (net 17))
 (segment (start 163.2964 86.7464) (end 163.2018 86.841) (width 0.2) (layer "B.Cu") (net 17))
 (segment (start 154.053 93.127) (end 158.92 97.994) (width 0.2) (layer "F.Cu") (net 7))
 (segment (start 158.92 97.994) (end 158.92 101.698) (width 0.2) (layer "F.Cu") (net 7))
 (segment (start 144.78 80.772) (end 143.945 80.772) (width 0.2) (layer "F.Cu") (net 7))
 (via (at 154.053 93.127) (size 0.6) (drill 0.3) (layers "F.Cu" "B.Cu") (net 7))
 (segment (start 147.932 93.127) (end 143.6716 88.8666) (width 0.2) (layer "B.Cu") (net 7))
 (segment (start 143.6716 81.8804) (end 144.78 80.772) (width 0.2) (layer "B.Cu") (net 7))
 (segment (start 154.053 93.127) (end 147.932 93.127) (width 0.2) (layer "B.Cu") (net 7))
 (segment (start 143.6716 88.8666) (end 143.6716 81.8804) (width 0.2) (layer "B.Cu") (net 7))
 (segment (start 163.5893 79.046) (end 163.5893 80.0843) (width 0.2) (layer "F.Cu") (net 5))
 (segment (start 142.3594 87.4397) (end 143.945 85.8541) (width 0.2) (layer "F.Cu") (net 5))
 (segment (start 164.4843 81.7641) (end 164.4843 80.7491) (width 0.2) (layer "F.Cu") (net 5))
 (segment (start 164.2541 80.7491) (end 164.4843 80.7491) (width 0.2) (layer "F.Cu") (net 5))
 (segment (start 164.4843 80.7491) (end 164.4843 81.7641) (width 0.2) (layer "F.Cu") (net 5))
 (segment (start 151.3 100.5463) (end 142.3594 91.6057) (width 0.2) (layer "F.Cu") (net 5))
 (segment (start 143.945 85.852) (end 144.78 85.852) (width 0.2) (layer "F.Cu") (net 5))
 (segment (start 164.592 74.977) (end 165.6152 76.0002) (width 0.2) (layer "F.Cu") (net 5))
 (segment (start 163.5893 80.0843) (end 164.2541 80.7491) (width 0.2) (layer "F.Cu") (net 5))
 (segment (start 143.945 85.8541) (end 143.945 85.852) (width 0.2) (layer "F.Cu") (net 5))
 (segment (start 165.6152 76.0002) (end 165.6152 78.1975) (width 0.2) (layer "F.Cu") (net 5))
 (segment (start 151.3 101.698) (end 151.3 100.5463) (width 0.2) (layer "F.Cu") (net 5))
 (segment (start 164.0961 78.5392) (end 163.5893 79.046) (width 0.2) (layer "F.Cu") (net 5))
 (segment (start 142.3594 91.6057) (end 142.3594 87.4397) (width 0.2) (layer "F.Cu") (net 5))
 (segment (start 165.2735 78.5392) (end 164.0961 78.5392) (width 0.2) (layer "F.Cu") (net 5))
 (segment (start 165.6152 78.1975) (end 165.2735 78.5392) (width 0.2) (layer "F.Cu") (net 5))
 (via (at 164.4843 80.7491) (size 0.6) (drill 0.3) (layers "F.Cu" "B.Cu") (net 5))
 (segment (start 165.4993 92.3877) (end 165.1159 92.7711) (width 0.2) (layer "B.Cu") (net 5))
 (segment (start 165.4993 81.7641) (end 165.4993 92.3877) (width 0.2) (layer "B.Cu") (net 5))
 (segment (start 165.1159 92.7711) (end 164.5146 92.7711) (width 0.2) (layer "B.Cu") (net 5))
 (segment (start 164.4843 80.7491) (end 164.4843 81.7641) (width 0.2) (layer "B.Cu") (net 5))
 (segment (start 162.0607 91.7291) (end 152.4517 101.3381) (width 0.2) (layer "B.Cu") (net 5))
 (segment (start 151.3 101.698) (end 152.4517 101.698) (width 0.2) (layer "B.Cu") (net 5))
 (segment (start 152.4517 101.3381) (end 152.4517 101.698) (width 0.2) (layer "B.Cu") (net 5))
 (segment (start 164.4843 80.7491) (end 165.4993 81.7641) (width 0.2) (layer "B.Cu") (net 5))
 (segment (start 164.5146 92.7711) (end 163.4726 91.7291) (width 0.2) (layer "B.Cu") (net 5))
 (segment (start 163.4726 91.7291) (end 162.0607 91.7291) (width 0.2) (layer "B.Cu") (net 5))
 (segment (start 164.4843 81.7641) (end 164.4843 80.7491) (width 0.2) (layer "B.Cu") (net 5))
 (segment (start 142.1571 87.038) (end 142.1931 87.038) (width 0.2) (layer "F.Cu") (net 3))
 (segment (start 142.3928 84.8642) (end 143.945 83.312) (width 0.2) (layer "F.Cu") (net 3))
 (segment (start 152.6883 101.9859) (end 151.8011 102.8731) (width 0.2) (layer "F.Cu") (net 3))
 (segment (start 163.1874 92.3506) (end 163.1874 87.7063) (width 0.2) (layer "F.Cu") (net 3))
 (segment (start 141.9571 92.3324) (end 141.9571 87.238) (width 0.2) (layer "F.Cu") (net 3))
 (segment (start 152.6883 101.698) (end 152.6883 101.9859) (width 0.2) (layer "F.Cu") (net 3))
 (segment (start 142.3928 86.8383) (end 142.3928 84.8642) (width 0.2) (layer "F.Cu") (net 3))
 (segment (start 163.1874 87.7063) (end 165.6403 85.2534) (width 0.2) (layer "F.Cu") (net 3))
 (segment (start 165.6403 85.2534) (end 165.6403 80.5973) (width 0.2) (layer "F.Cu") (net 3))
 (segment (start 153.84 101.698) (end 152.6883 101.698) (width 0.2) (layer "F.Cu") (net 3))
 (segment (start 165.6403 80.5973) (end 164.592 79.549) (width 0.2) (layer "F.Cu") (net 3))
 (segment (start 144.78 83.312) (end 143.945 83.312) (width 0.2) (layer "F.Cu") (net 3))
 (segment (start 151.8011 102.8731) (end 150.8401 102.8731) (width 0.2) (layer "F.Cu") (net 3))
 (segment (start 150.03 100.4053) (end 141.9571 92.3324) (width 0.2) (layer "F.Cu") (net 3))
 (segment (start 150.8401 102.8731) (end 150.03 102.063) (width 0.2) (layer "F.Cu") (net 3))
 (segment (start 150.03 102.063) (end 150.03 100.4053) (width 0.2) (layer "F.Cu") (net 3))
 (segment (start 142.1931 87.038) (end 142.3928 86.8383) (width 0.2) (layer "F.Cu") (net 3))
 (segment (start 141.9571 87.238) (end 142.1571 87.038) (width 0.2) (layer "F.Cu") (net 3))
 (via (at 163.1874 92.3506) (size 0.6) (drill 0.3) (layers "F.Cu" "B.Cu") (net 3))
 (segment (start 153.84 100.5463) (end 154.9917 100.5463) (width 0.2) (layer "B.Cu") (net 3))
 (segment (start 163.1874 92.3506) (end 163.1858 92.3506) (width 0.2) (layer "B.Cu") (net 3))
 (segment (start 153.84 101.698) (end 153.84 100.5463) (width 0.2) (layer "B.Cu") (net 3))
 (segment (start 163.1858 92.3506) (end 163.1874 92.3506) (width 0.2) (layer "B.Cu") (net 3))
 (segment (start 154.9917 100.5463) (end 163.1874 92.3506) (width 0.2) (layer "B.Cu") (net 3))
 (segment (start 141.9571 86.67) (end 140.1115 88.5156) (width 0.2) (layer "F.Cu") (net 6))
 (segment (start 141.9571 80.2199) (end 141.9571 86.67) (width 0.2) (layer "F.Cu") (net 6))
 (segment (start 144.78 78.232) (end 143.945 78.232) (width 0.2) (layer "F.Cu") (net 6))
 (segment (start 140.1115 101.7401) (end 144.0328 105.6614) (width 0.2) (layer "F.Cu") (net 6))
 (segment (start 143.945 78.232) (end 141.9571 80.2199) (width 0.2) (layer "F.Cu") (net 6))
 (segment (start 144.0328 105.6614) (end 144.0328 108.5887) (width 0.2) (layer "F.Cu") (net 6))
 (segment (start 140.1115 88.5156) (end 140.1115 101.7401) (width 0.2) (layer "F.Cu") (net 6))
 (via (at 144.0328 108.5887) (size 0.6) (drill 0.3) (layers "F.Cu" "B.Cu") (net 6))
 (segment (start 148.6061 108.5887) (end 155.2283 101.9665) (width 0.2) (layer "B.Cu") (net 6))
 (segment (start 156.38 101.698) (end 155.2283 101.698) (width 0.2) (layer "B.Cu") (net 6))
 (segment (start 144.0328 108.5887) (end 148.6061 108.5887) (width 0.2) (layer "B.Cu") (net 6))
 (segment (start 155.2283 101.9665) (end 155.2283 101.698) (width 0.2) (layer "B.Cu") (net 6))
 (segment (start 144.78 75.692) (end 143.945 75.692) (width 0.2) (layer "F.Cu") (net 2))
 (segment (start 141.5247 78.1123) (end 141.5247 85.5513) (width 0.2) (layer "F.Cu") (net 2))
 (segment (start 140.4925 72.2395) (end 143.945 75.692) (width 0.2) (layer "F.Cu") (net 2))
 (segment (start 140.208 72.2395) (end 140.4925 72.2395) (width 0.2) (layer "F.Cu") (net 2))
 (segment (start 143.945 75.692) (end 141.5247 78.1123) (width 0.2) (layer "F.Cu") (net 2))
 (segment (start 141.5247 85.5513) (end 140.208 86.868) (width 0.2) (layer "F.Cu") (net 2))
 (segment (start 141.224 107.7783) (end 140.5457 107.7783) (width 0.2) (layer "F.Cu") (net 8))
 (segment (start 141.224 108.68) (end 141.224 107.7783) (width 0.2) (layer "F.Cu") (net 8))
 (segment (start 139.1819 86.0691) (end 140.208 85.043) (width 0.2) (layer "F.Cu") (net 8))
 (segment (start 139.1819 106.4145) (end 139.1819 86.0691) (width 0.2) (layer "F.Cu") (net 8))
 (segment (start 140.5457 107.7783) (end 139.1819 106.4145) (width 0.2) (layer "F.Cu") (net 8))
 (segment (start 140.208 85.043) (end 140.208 81.031) (width 0.2) (layer "F.Cu") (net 8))
 (segment (start 160.0717 93.1265) (end 162.4088 90.7894) (width 0.2) (layer "F.Cu") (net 14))
 (segment (start 162.4088 84.8658) (end 160.855 83.312) (width 0.2) (layer "F.Cu") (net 14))
 (segment (start 149.758 105.796) (end 156.058 105.796) (width 0.2) (layer "F.Cu") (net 14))
 (segment (start 156.058 105.796) (end 157.2097 105.796) (width 0.2) (layer "F.Cu") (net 14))
 (segment (start 160.855 83.312) (end 160.02 83.312) (width 0.2) (layer "F.Cu") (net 14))
 (segment (start 157.2097 105.796) (end 160.0717 102.934) (width 0.2) (layer "F.Cu") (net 14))
 (segment (start 160.0717 102.934) (end 160.0717 93.1265) (width 0.2) (layer "F.Cu") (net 14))
 (segment (start 162.4088 90.7894) (end 162.4088 84.8658) (width 0.2) (layer "F.Cu") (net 14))
 (segment (start 162.887 82.804) (end 160.855 80.772) (width 0.2) (layer "F.Cu") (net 15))
 (segment (start 160.855 80.772) (end 160.02 80.772) (width 0.2) (layer "F.Cu") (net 15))
 (segment (start 164.592 82.804) (end 162.887 82.804) (width 0.2) (layer "F.Cu") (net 15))
 (segment (start 144.78 73.152) (end 143.945 73.152) (width 0.2) (layer "F.Cu") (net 10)))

